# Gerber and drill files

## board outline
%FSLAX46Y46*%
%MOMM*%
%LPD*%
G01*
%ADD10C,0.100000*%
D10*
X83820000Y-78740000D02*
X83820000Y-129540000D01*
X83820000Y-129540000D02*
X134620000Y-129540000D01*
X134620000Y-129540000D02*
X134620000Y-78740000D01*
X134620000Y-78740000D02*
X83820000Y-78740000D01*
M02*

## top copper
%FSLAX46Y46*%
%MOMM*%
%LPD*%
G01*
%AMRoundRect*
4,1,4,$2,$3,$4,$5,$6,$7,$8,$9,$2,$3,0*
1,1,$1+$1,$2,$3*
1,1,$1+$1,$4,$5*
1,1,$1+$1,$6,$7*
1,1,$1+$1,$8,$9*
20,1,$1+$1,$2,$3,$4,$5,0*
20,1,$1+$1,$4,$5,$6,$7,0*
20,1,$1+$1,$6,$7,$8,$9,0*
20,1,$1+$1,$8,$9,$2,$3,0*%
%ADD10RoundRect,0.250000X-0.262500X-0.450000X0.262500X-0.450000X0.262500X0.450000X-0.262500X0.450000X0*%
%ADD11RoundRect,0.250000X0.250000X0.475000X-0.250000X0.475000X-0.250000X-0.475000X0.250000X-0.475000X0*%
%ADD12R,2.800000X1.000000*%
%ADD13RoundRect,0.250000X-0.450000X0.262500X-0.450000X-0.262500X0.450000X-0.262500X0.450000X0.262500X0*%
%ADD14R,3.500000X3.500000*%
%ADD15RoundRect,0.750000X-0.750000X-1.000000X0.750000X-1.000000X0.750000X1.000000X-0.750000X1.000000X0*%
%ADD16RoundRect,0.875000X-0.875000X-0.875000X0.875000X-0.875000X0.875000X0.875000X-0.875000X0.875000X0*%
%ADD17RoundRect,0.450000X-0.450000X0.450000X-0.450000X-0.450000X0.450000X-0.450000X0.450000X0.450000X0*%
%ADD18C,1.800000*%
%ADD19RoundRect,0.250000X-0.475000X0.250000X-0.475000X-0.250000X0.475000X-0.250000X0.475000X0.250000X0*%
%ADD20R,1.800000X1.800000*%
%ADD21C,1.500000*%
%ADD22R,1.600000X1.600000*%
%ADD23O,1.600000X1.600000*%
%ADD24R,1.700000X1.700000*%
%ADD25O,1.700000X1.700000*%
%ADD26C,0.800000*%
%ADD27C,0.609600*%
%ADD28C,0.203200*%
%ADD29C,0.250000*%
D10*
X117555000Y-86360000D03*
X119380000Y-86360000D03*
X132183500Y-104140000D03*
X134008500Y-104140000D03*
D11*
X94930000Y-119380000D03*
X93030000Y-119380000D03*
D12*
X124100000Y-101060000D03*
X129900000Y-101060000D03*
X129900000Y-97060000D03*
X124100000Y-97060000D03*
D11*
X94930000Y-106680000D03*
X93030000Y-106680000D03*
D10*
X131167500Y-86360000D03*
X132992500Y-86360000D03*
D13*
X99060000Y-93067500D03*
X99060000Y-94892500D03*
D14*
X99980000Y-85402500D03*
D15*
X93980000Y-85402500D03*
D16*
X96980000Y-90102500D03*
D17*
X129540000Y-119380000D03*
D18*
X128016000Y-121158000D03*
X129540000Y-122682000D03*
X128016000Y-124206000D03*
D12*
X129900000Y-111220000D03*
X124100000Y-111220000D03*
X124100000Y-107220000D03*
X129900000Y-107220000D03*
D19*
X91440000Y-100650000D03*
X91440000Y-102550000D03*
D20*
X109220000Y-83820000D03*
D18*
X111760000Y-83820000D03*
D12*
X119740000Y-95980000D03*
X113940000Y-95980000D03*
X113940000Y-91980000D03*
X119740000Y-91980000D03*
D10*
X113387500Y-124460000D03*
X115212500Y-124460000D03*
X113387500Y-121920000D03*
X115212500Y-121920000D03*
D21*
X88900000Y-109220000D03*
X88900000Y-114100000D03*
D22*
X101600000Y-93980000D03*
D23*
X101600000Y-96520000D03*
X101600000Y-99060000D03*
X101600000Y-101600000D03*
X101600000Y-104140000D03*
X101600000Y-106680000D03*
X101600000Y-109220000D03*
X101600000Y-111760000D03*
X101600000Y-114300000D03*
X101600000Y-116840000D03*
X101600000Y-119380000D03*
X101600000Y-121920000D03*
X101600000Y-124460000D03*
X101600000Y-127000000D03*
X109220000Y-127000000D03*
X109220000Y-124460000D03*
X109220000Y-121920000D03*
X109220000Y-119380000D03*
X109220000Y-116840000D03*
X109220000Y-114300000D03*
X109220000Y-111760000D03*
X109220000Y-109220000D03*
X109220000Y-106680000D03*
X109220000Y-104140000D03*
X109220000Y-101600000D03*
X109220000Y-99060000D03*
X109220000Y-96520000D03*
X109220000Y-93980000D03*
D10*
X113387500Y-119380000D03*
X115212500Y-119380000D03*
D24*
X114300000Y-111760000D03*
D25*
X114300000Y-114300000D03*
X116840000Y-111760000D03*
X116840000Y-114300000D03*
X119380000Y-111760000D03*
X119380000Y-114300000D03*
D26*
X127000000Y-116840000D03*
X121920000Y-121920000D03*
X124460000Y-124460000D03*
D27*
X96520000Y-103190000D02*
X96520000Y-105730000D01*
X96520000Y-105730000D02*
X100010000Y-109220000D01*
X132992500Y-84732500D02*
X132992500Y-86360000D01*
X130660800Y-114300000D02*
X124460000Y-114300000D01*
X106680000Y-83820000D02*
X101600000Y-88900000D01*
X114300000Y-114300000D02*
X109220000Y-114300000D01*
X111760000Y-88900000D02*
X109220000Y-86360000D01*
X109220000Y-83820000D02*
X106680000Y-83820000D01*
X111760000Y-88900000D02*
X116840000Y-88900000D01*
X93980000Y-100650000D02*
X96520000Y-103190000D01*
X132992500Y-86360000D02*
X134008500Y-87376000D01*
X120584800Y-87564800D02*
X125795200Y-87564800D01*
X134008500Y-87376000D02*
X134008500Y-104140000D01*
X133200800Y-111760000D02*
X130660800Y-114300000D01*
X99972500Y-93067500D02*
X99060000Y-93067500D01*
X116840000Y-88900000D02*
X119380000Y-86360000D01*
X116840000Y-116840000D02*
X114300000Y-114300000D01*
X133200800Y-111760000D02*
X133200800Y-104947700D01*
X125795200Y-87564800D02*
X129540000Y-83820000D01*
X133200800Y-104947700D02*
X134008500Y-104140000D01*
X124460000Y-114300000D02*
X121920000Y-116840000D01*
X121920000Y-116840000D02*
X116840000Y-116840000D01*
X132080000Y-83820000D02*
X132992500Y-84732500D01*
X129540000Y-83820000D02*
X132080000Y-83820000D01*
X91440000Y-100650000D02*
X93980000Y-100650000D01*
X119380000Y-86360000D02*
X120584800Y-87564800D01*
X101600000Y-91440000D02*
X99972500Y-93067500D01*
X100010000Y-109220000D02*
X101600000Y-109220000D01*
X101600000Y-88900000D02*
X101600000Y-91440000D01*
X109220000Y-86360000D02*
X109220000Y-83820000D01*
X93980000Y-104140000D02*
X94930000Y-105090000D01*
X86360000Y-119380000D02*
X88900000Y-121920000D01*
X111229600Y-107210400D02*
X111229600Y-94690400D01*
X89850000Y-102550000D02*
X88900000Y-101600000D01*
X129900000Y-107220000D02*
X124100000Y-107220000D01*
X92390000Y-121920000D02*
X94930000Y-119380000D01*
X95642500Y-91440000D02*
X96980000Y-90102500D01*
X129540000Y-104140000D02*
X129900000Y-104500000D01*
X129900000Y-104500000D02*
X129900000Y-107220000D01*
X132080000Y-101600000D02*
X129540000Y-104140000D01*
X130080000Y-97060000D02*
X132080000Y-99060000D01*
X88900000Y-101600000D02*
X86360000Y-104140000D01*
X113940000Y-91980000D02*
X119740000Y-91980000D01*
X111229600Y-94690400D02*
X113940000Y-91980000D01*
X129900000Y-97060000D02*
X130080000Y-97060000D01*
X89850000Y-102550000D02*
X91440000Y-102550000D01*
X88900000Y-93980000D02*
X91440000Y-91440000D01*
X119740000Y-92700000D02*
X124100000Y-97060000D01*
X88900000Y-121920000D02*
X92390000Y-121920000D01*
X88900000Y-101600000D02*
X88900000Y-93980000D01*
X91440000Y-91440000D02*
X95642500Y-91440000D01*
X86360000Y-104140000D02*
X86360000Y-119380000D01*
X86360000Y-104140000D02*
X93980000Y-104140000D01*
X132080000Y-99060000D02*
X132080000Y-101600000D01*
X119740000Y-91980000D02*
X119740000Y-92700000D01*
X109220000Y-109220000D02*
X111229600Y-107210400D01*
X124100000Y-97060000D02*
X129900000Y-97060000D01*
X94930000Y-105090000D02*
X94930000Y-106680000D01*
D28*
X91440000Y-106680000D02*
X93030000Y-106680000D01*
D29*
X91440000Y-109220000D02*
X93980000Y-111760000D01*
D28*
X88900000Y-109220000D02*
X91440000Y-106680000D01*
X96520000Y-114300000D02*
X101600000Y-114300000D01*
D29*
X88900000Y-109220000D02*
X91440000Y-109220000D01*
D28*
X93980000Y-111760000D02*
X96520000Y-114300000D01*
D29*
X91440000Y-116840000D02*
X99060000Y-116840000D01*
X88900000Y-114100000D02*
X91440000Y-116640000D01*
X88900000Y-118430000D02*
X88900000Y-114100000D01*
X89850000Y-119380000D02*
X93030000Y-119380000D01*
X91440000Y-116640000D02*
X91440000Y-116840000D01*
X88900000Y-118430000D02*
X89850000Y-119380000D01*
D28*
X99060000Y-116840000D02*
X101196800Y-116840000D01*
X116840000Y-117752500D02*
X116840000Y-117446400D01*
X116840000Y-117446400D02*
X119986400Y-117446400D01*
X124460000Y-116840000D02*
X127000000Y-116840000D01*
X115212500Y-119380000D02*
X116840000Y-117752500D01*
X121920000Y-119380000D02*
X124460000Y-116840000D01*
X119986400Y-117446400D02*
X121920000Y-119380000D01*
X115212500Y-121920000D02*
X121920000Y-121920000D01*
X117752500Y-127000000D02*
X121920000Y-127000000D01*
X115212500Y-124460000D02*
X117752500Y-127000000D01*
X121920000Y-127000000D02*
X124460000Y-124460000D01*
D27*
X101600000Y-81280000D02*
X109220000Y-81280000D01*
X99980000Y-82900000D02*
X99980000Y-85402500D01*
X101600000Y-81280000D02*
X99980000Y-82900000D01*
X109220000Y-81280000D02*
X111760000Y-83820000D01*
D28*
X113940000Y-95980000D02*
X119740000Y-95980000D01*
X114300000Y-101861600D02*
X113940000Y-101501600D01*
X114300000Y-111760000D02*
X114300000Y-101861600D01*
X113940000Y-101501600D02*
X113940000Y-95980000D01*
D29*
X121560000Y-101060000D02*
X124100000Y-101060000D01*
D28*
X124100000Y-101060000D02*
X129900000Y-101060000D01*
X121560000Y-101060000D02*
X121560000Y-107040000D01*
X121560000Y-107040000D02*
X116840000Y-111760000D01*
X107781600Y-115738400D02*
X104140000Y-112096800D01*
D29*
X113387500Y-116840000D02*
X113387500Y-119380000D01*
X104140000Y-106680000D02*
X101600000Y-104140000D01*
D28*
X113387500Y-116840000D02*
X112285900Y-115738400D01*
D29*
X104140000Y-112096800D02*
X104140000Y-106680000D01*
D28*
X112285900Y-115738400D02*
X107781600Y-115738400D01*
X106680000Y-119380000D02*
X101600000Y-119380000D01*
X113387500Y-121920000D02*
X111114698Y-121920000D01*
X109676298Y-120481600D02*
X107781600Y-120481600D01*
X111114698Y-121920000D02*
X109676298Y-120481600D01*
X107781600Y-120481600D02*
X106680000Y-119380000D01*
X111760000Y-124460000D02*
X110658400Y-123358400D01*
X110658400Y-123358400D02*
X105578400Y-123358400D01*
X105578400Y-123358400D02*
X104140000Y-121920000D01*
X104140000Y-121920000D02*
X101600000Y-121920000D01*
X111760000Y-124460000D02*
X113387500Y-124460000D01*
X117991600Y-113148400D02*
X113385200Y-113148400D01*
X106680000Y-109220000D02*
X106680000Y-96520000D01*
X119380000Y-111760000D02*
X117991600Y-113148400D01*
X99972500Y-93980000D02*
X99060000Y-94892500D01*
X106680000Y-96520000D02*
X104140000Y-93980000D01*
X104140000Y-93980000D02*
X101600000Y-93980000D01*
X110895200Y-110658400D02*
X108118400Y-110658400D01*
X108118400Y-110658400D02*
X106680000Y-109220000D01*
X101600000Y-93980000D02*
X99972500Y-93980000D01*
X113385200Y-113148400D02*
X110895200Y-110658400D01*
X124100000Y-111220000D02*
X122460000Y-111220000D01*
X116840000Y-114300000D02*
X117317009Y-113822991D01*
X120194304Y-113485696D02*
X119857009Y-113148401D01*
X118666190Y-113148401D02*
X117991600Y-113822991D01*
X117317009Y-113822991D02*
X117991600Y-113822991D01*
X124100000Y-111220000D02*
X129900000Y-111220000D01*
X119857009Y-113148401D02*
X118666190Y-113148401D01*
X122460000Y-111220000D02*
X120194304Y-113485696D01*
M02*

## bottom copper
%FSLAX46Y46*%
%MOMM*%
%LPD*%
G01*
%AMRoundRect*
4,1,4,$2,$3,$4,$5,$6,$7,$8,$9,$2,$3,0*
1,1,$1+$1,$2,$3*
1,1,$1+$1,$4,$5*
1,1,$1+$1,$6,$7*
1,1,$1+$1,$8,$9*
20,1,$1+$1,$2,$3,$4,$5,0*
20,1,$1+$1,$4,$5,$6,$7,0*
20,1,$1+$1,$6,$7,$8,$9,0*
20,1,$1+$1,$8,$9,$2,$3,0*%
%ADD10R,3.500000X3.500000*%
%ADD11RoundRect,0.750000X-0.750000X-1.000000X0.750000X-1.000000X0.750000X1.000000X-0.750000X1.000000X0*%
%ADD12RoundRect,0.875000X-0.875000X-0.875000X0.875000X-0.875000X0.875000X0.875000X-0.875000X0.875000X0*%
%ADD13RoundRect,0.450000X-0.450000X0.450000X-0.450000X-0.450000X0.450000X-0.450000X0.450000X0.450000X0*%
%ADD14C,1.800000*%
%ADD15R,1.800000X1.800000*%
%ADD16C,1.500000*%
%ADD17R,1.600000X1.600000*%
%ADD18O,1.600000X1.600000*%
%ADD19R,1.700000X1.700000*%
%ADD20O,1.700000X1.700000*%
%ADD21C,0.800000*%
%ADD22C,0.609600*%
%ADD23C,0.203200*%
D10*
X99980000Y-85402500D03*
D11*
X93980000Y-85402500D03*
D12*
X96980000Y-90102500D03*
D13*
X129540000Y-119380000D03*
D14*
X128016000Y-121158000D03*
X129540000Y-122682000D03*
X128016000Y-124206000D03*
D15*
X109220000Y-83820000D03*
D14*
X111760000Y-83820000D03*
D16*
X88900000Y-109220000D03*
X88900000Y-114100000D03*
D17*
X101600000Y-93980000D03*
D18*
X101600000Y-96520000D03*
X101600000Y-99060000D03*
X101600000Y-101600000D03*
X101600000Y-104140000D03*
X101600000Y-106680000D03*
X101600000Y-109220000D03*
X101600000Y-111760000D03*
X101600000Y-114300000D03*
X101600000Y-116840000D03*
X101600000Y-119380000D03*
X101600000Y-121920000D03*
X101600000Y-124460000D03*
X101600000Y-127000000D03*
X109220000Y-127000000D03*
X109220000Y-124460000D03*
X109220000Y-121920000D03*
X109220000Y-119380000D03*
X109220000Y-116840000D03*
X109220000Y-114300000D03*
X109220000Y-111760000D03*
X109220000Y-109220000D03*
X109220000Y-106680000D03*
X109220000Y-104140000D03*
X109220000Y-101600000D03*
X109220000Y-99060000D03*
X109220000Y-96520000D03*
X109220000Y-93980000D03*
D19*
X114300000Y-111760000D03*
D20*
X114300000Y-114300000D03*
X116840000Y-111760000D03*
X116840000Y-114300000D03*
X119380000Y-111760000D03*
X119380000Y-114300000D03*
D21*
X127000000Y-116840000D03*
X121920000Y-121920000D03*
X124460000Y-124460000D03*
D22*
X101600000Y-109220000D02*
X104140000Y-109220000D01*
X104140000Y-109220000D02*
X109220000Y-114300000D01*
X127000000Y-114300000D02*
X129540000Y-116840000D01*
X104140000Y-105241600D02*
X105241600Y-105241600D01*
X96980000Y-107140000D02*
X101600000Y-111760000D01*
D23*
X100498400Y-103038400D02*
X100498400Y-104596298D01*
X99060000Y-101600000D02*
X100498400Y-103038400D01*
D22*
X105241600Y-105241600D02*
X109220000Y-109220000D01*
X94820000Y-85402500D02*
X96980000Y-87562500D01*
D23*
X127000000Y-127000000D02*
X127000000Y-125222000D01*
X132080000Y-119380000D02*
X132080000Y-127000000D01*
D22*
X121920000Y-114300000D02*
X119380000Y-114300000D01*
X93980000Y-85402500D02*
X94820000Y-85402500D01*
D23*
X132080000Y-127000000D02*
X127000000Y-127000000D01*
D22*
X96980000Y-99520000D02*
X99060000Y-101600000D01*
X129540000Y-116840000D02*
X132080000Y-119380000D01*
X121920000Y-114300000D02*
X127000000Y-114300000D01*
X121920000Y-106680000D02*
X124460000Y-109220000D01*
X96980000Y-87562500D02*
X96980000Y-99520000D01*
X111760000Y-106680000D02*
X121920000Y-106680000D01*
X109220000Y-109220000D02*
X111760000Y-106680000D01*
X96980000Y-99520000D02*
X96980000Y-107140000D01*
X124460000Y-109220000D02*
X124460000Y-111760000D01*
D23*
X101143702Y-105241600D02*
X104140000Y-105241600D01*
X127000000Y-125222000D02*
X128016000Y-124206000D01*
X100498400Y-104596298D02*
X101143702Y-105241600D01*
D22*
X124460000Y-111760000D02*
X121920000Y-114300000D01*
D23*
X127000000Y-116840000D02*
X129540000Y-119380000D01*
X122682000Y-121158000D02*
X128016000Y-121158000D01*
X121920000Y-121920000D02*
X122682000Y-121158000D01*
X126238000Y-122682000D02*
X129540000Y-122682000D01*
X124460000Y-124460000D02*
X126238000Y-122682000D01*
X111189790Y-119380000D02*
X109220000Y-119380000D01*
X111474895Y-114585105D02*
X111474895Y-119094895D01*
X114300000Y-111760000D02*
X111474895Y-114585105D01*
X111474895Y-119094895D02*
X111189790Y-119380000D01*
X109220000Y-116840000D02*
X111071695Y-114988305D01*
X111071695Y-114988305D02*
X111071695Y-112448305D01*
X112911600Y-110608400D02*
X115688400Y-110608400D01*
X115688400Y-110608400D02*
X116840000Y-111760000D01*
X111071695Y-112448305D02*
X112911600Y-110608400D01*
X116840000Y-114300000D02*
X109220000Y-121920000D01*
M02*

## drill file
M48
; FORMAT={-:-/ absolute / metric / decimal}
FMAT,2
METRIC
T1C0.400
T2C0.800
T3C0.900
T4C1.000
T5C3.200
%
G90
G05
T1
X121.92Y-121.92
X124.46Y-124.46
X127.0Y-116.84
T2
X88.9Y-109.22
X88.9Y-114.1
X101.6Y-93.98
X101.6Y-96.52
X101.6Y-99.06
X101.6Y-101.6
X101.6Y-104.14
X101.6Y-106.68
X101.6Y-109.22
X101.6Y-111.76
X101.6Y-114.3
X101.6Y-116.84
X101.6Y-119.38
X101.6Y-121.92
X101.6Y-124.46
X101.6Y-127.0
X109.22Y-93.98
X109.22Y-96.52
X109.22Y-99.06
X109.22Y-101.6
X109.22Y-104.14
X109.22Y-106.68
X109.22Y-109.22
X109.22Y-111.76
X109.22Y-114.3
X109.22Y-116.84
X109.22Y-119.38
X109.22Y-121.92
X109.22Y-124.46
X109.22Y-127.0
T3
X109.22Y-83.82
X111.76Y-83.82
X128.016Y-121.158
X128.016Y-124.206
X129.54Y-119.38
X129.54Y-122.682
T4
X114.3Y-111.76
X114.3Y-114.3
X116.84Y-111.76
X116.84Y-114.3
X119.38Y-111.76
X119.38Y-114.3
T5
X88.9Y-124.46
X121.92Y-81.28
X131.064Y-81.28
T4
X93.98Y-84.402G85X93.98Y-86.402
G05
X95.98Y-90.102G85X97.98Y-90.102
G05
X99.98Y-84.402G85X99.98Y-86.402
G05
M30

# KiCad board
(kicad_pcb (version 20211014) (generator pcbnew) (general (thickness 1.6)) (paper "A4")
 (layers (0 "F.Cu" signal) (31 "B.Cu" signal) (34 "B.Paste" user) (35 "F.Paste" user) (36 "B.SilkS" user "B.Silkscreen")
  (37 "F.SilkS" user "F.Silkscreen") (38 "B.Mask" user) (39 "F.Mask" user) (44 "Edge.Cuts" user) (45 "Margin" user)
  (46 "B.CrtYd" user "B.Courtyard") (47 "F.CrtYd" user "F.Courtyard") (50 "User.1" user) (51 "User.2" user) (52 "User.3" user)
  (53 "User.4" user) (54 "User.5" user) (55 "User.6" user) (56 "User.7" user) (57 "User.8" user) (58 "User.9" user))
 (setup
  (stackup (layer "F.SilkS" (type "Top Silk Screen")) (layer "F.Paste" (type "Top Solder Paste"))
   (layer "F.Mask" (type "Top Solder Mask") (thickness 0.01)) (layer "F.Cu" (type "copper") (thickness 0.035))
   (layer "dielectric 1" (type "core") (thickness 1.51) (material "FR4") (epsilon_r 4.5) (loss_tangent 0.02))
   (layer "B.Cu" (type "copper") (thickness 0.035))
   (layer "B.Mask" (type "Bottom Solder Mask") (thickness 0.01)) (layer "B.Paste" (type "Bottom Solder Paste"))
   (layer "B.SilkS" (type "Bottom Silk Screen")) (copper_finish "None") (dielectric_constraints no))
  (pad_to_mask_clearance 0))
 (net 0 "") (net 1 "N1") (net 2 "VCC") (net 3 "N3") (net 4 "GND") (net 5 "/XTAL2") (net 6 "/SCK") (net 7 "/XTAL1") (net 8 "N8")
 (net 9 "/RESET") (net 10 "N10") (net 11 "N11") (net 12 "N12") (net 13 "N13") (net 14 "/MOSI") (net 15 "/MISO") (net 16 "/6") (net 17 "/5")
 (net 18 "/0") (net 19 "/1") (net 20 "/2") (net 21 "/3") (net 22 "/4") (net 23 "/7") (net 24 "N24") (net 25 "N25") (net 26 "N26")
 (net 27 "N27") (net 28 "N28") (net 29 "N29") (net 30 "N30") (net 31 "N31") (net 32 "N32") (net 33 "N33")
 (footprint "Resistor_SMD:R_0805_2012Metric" (layer "F.Cu") (at 118.4675 86.36)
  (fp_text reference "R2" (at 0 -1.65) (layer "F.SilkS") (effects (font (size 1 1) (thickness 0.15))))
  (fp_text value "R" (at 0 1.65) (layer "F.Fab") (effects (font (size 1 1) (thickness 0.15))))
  (pad "1" smd roundrect (at -0.9125 0) (size 1.025 1.4) (layers "F.Cu" "F.Paste" "F.Mask") (roundrect_rratio 0.243902) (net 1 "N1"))
  (pad "2" smd roundrect (at 0.9125 0) (size 1.025 1.4) (layers "F.Cu" "F.Paste" "F.Mask") (roundrect_rratio 0.243902) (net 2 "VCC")))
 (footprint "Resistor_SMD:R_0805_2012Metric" (layer "F.Cu") (at 133.096 104.14)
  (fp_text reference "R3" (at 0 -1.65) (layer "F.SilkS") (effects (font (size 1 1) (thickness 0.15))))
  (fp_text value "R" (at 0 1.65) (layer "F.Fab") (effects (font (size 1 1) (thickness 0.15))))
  (pad "1" smd roundrect (at -0.9125 0) (size 1.025 1.4) (layers "F.Cu" "F.Paste" "F.Mask") (roundrect_rratio 0.243902) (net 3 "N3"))
  (pad "2" smd roundrect (at 0.9125 0) (size 1.025 1.4) (layers "F.Cu" "F.Paste" "F.Mask") (roundrect_rratio 0.243902) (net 2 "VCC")))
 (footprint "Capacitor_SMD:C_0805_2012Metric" (layer "F.Cu") (at 93.98 119.38 180)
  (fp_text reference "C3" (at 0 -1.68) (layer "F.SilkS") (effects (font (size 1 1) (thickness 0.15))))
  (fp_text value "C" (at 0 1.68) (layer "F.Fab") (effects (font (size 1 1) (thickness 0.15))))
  (pad "1" smd roundrect (at -0.95 0 180) (size 1 1.45) (layers "F.Cu" "F.Paste" "F.Mask") (roundrect_rratio 0.25) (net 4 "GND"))
  (pad "2" smd roundrect (at 0.95 0 180) (size 1 1.45) (layers "F.Cu" "F.Paste" "F.Mask") (roundrect_rratio 0.25) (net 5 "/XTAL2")))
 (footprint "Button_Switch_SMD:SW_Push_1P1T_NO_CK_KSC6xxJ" (layer "F.Cu") (at 127 99.06 180)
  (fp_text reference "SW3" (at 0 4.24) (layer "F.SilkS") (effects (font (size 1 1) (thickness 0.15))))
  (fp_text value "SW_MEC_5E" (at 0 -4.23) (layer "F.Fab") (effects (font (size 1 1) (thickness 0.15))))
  (pad "1" smd rect (at 2.9 -2 180) (size 2.8 1) (layers "F.Cu" "F.Paste" "F.Mask") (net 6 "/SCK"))
  (pad "1" smd rect (at -2.9 -2 180) (size 2.8 1) (layers "F.Cu" "F.Paste" "F.Mask") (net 6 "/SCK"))
  (pad "2" smd rect (at -2.9 2 180) (size 2.8 1) (layers "F.Cu" "F.Paste" "F.Mask") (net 4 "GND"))
  (pad "2" smd rect (at 2.9 2 180) (size 2.8 1) (layers "F.Cu" "F.Paste" "F.Mask") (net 4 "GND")))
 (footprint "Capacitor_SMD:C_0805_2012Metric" (layer "F.Cu") (at 93.98 106.68 180)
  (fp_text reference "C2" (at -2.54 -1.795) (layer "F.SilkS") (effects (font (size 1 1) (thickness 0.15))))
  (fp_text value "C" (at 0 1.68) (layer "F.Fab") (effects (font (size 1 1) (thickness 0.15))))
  (pad "1" smd roundrect (at -0.95 0 180) (size 1 1.45) (layers "F.Cu" "F.Paste" "F.Mask") (roundrect_rratio 0.25) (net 4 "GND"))
  (pad "2" smd roundrect (at 0.95 0 180) (size 1 1.45) (layers "F.Cu" "F.Paste" "F.Mask") (roundrect_rratio 0.25) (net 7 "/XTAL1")))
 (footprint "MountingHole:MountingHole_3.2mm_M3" (layer "F.Cu") (at 121.92 81.28)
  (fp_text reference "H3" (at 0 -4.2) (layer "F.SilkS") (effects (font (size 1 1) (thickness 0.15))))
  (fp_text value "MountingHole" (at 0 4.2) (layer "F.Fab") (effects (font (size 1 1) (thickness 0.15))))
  (pad "" np_thru_hole circle (at 0 0) (size 3.2 3.2) (drill 3.2) (layers *.Cu *.Mask)))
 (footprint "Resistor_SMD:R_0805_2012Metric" (layer "F.Cu") (at 132.08 86.36)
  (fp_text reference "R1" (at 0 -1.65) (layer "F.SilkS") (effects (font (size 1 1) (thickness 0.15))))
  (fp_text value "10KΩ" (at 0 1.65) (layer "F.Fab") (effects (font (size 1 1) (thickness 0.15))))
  (pad "1" smd roundrect (at -0.9125 0) (size 1.025 1.4) (layers "F.Cu" "F.Paste" "F.Mask") (roundrect_rratio 0.243902) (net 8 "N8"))
  (pad "2" smd roundrect (at 0.9125 0) (size 1.025 1.4) (layers "F.Cu" "F.Paste" "F.Mask") (roundrect_rratio 0.243902) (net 2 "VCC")))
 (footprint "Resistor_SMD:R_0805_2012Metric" (layer "F.Cu") (at 99.06 93.98 -90)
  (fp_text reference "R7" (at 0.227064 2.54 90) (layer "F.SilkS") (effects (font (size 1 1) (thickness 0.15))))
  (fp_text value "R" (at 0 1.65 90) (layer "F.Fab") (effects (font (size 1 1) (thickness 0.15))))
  (pad "1" smd roundrect (at -0.9125 0 270) (size 1.025 1.4) (layers "F.Cu" "F.Paste" "F.Mask") (roundrect_rratio 0.243902) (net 2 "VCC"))
  (pad "2" smd roundrect (at 0.9125 0 270) (size 1.025 1.4) (layers "F.Cu" "F.Paste" "F.Mask") (roundrect_rratio 0.243902) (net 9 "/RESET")))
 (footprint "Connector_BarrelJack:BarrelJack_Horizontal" (layer "F.Cu") (at 99.98 85.4025)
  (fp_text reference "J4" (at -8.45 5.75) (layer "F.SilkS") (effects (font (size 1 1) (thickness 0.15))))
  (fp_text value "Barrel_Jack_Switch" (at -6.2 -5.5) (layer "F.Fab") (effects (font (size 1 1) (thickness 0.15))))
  (pad "1" thru_hole rect (at 0 0) (size 3.5 3.5) (drill oval 1 3) (layers *.Cu *.Mask) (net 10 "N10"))
  (pad "2" thru_hole roundrect (at -6 0) (size 3 3.5) (drill oval 1 3) (layers *.Cu *.Mask) (roundrect_rratio 0.25) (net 4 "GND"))
  (pad "3" thru_hole roundrect (at -3 4.7) (size 3.5 3.5) (drill oval 3 1) (layers *.Cu *.Mask) (roundrect_rratio 0.25) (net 4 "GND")))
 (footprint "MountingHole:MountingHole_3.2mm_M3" (layer "F.Cu") (at 88.9 124.46)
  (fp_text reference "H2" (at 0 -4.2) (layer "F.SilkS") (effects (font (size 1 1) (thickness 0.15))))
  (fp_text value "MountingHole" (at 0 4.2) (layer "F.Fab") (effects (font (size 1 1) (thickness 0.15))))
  (pad "" np_thru_hole circle (at 0 0) (size 3.2 3.2) (drill 3.2) (layers *.Cu *.Mask)))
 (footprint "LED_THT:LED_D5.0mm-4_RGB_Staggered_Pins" (layer "F.Cu") (at 129.54 119.38 -90)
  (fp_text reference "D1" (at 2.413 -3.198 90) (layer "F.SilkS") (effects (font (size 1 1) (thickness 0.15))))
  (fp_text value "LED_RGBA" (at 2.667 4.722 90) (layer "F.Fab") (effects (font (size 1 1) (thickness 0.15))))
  (pad "1" thru_hole roundrect (at 0 0 270) (size 1.8 1.8) (drill 0.9) (layers *.Cu *.Mask) (roundrect_rratio 0.25) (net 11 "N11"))
  (pad "2" thru_hole circle (at 1.778 1.524 270) (size 1.8 1.8) (drill 0.9) (layers *.Cu *.Mask) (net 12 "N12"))
  (pad "3" thru_hole circle (at 3.302 0 270) (size 1.8 1.8) (drill 0.9) (layers *.Cu *.Mask) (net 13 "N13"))
  (pad "4" thru_hole circle (at 4.826 1.524 270) (size 1.8 1.8) (drill 0.9) (layers *.Cu *.Mask) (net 4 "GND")))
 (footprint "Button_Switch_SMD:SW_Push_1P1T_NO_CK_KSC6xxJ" (layer "F.Cu") (at 127 109.22 180)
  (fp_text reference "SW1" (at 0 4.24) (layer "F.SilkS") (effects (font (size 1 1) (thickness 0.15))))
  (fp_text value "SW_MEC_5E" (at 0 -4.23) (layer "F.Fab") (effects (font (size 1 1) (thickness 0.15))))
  (pad "1" smd rect (at -2.9 -2 180) (size 2.8 1) (layers "F.Cu" "F.Paste" "F.Mask") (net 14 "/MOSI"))
  (pad "1" smd rect (at 2.9 -2 180) (size 2.8 1) (layers "F.Cu" "F.Paste" "F.Mask") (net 14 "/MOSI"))
  (pad "2" smd rect (at 2.9 2 180) (size 2.8 1) (layers "F.Cu" "F.Paste" "F.Mask") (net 4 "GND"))
  (pad "2" smd rect (at -2.9 2 180) (size 2.8 1) (layers "F.Cu" "F.Paste" "F.Mask") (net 4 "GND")))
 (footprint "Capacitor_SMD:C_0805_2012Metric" (layer "F.Cu") (at 91.44 101.6 -90)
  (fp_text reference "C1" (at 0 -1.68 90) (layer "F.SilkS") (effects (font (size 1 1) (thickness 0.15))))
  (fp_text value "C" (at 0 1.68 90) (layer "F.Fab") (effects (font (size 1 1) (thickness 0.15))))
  (pad "1" smd roundrect (at -0.95 0 270) (size 1 1.45) (layers "F.Cu" "F.Paste" "F.Mask") (roundrect_rratio 0.25) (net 2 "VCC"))
  (pad "2" smd roundrect (at 0.95 0 270) (size 1 1.45) (layers "F.Cu" "F.Paste" "F.Mask") (roundrect_rratio 0.25) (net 4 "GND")))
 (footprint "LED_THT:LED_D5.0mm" (layer "F.Cu") (at 109.22 83.82)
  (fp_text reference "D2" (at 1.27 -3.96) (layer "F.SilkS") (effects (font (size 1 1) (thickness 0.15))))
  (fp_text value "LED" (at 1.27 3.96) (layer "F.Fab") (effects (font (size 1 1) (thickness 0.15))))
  (pad "1" thru_hole rect (at 0 0) (size 1.8 1.8) (drill 0.9) (layers *.Cu *.Mask) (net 2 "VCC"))
  (pad "2" thru_hole circle (at 2.54 0) (size 1.8 1.8) (drill 0.9) (layers *.Cu *.Mask) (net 10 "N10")))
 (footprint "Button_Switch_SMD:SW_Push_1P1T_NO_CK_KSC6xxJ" (layer "F.Cu") (at 116.84 93.98 180)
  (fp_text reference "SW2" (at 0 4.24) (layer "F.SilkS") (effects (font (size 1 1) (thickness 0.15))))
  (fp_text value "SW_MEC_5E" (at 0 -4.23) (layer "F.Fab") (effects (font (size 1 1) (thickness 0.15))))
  (pad "1" smd rect (at -2.9 -2 180) (size 2.8 1) (layers "F.Cu" "F.Paste" "F.Mask") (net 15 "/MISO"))
  (pad "1" smd rect (at 2.9 -2 180) (size 2.8 1) (layers "F.Cu" "F.Paste" "F.Mask") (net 15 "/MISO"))
  (pad "2" smd rect (at 2.9 2 180) (size 2.8 1) (layers "F.Cu" "F.Paste" "F.Mask") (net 4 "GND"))
  (pad "2" smd rect (at -2.9 2 180) (size 2.8 1) (layers "F.Cu" "F.Paste" "F.Mask") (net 4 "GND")))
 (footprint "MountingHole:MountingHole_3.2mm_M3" (layer "F.Cu") (at 131.064 81.28)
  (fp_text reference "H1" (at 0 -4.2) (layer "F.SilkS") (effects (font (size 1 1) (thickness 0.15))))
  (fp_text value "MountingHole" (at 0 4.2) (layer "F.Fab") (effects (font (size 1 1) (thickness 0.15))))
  (pad "" np_thru_hole circle (at 0 0) (size 3.2 3.2) (drill 3.2) (layers *.Cu *.Mask)))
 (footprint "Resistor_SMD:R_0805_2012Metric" (layer "F.Cu") (at 114.3 124.46)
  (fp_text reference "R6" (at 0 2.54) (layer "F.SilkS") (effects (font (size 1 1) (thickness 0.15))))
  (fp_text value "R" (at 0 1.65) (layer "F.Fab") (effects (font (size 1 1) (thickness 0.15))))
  (pad "1" smd roundrect (at -0.9125 0) (size 1.025 1.4) (layers "F.Cu" "F.Paste" "F.Mask") (roundrect_rratio 0.243902) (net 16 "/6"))
  (pad "2" smd roundrect (at 0.9125 0) (size 1.025 1.4) (layers "F.Cu" "F.Paste" "F.Mask") (roundrect_rratio 0.243902) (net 13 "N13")))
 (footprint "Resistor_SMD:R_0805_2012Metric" (layer "F.Cu") (at 114.3 121.92)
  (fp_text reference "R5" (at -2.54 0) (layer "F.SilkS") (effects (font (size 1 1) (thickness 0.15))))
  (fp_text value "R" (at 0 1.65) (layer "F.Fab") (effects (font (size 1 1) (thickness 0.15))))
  (pad "1" smd roundrect (at -0.9125 0) (size 1.025 1.4) (layers "F.Cu" "F.Paste" "F.Mask") (roundrect_rratio 0.243902) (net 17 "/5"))
  (pad "2" smd roundrect (at 0.9125 0) (size 1.025 1.4) (layers "F.Cu" "F.Paste" "F.Mask") (roundrect_rratio 0.243902) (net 12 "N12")))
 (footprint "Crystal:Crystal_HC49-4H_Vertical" (layer "F.Cu") (at 88.9 109.22 -90)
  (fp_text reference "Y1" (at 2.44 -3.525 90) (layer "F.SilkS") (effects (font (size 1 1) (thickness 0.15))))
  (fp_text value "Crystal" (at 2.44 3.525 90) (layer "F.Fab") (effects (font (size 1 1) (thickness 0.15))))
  (pad "1" thru_hole circle (at 0 0 270) (size 1.5 1.5) (drill 0.8) (layers *.Cu *.Mask) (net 7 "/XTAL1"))
  (pad "2" thru_hole circle (at 4.88 0 270) (size 1.5 1.5) (drill 0.8) (layers *.Cu *.Mask) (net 5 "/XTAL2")))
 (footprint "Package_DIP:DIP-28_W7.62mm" (layer "F.Cu") (at 101.6 93.98)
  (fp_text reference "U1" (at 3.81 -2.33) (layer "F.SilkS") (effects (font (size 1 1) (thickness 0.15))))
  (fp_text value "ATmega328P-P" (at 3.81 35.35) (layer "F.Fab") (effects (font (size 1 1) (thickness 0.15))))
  (pad "1" thru_hole rect (at 0 0) (size 1.6 1.6) (drill 0.8) (layers *.Cu *.Mask) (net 9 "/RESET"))
  (pad "2" thru_hole oval (at 0 2.54) (size 1.6 1.6) (drill 0.8) (layers *.Cu *.Mask) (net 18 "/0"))
  (pad "3" thru_hole oval (at 0 5.08) (size 1.6 1.6) (drill 0.8) (layers *.Cu *.Mask) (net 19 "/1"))
  (pad "4" thru_hole oval (at 0 7.62) (size 1.6 1.6) (drill 0.8) (layers *.Cu *.Mask) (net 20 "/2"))
  (pad "5" thru_hole oval (at 0 10.16) (size 1.6 1.6) (drill 0.8) (layers *.Cu *.Mask) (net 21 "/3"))
  (pad "6" thru_hole oval (at 0 12.7) (size 1.6 1.6) (drill 0.8) (layers *.Cu *.Mask) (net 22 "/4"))
  (pad "7" thru_hole oval (at 0 15.24) (size 1.6 1.6) (drill 0.8) (layers *.Cu *.Mask) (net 2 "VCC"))
  (pad "8" thru_hole oval (at 0 17.78) (size 1.6 1.6) (drill 0.8) (layers *.Cu *.Mask) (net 4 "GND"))
  (pad "9" thru_hole oval (at 0 20.32) (size 1.6 1.6) (drill 0.8) (layers *.Cu *.Mask) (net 7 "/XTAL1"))
  (pad "10" thru_hole oval (at 0 22.86) (size 1.6 1.6) (drill 0.8) (layers *.Cu *.Mask) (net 5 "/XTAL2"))
  (pad "11" thru_hole oval (at 0 25.4) (size 1.6 1.6) (drill 0.8) (layers *.Cu *.Mask) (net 17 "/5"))
  (pad "12" thru_hole oval (at 0 27.94) (size 1.6 1.6) (drill 0.8) (layers *.Cu *.Mask) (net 16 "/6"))
  (pad "13" thru_hole oval (at 0 30.48) (size 1.6 1.6) (drill 0.8) (layers *.Cu *.Mask) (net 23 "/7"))
  (pad "14" thru_hole oval (at 0 33.02) (size 1.6 1.6) (drill 0.8) (layers *.Cu *.Mask) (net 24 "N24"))
  (pad "15" thru_hole oval (at 7.62 33.02) (size 1.6 1.6) (drill 0.8) (layers *.Cu *.Mask) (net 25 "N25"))
  (pad "16" thru_hole oval (at 7.62 30.48) (size 1.6 1.6) (drill 0.8) (layers *.Cu *.Mask) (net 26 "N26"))
  (pad "17" thru_hole oval (at 7.62 27.94) (size 1.6 1.6) (drill 0.8) (layers *.Cu *.Mask) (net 14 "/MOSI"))
  (pad "18" thru_hole oval (at 7.62 25.4) (size 1.6 1.6) (drill 0.8) (layers *.Cu *.Mask) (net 15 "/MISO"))
  (pad "19" thru_hole oval (at 7.62 22.86) (size 1.6 1.6) (drill 0.8) (layers *.Cu *.Mask) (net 6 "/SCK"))
  (pad "20" thru_hole oval (at 7.62 20.32) (size 1.6 1.6) (drill 0.8) (layers *.Cu *.Mask) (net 2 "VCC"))
  (pad "21" thru_hole oval (at 7.62 17.78) (size 1.6 1.6) (drill 0.8) (layers *.Cu *.Mask) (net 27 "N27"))
  (pad "22" thru_hole oval (at 7.62 15.24) (size 1.6 1.6) (drill 0.8) (layers *.Cu *.Mask) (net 4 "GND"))
  (pad "23" thru_hole oval (at 7.62 12.7) (size 1.6 1.6) (drill 0.8) (layers *.Cu *.Mask) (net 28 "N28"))
  (pad "24" thru_hole oval (at 7.62 10.16) (size 1.6 1.6) (drill 0.8) (layers *.Cu *.Mask) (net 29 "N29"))
  (pad "25" thru_hole oval (at 7.62 7.62) (size 1.6 1.6) (drill 0.8) (layers *.Cu *.Mask) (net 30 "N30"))
  (pad "26" thru_hole oval (at 7.62 5.08) (size 1.6 1.6) (drill 0.8) (layers *.Cu *.Mask) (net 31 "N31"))
  (pad "27" thru_hole oval (at 7.62 2.54) (size 1.6 1.6) (drill 0.8) (layers *.Cu *.Mask) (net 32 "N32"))
  (pad "28" thru_hole oval (at 7.62 0) (size 1.6 1.6) (drill 0.8) (layers *.Cu *.Mask) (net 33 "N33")))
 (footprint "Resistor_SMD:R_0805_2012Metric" (layer "F.Cu") (at 114.3 119.38)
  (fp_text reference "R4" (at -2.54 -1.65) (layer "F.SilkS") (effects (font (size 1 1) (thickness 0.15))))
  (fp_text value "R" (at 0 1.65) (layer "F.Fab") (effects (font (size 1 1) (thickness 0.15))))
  (pad "1" smd roundrect (at -0.9125 0) (size 1.025 1.4) (layers "F.Cu" "F.Paste" "F.Mask") (roundrect_rratio 0.243902) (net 21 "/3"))
  (pad "2" smd roundrect (at 0.9125 0) (size 1.025 1.4) (layers "F.Cu" "F.Paste" "F.Mask") (roundrect_rratio 0.243902) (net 11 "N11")))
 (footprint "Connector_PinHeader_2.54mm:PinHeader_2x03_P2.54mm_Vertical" (layer "B.Cu") (at 114.3 111.76 -90)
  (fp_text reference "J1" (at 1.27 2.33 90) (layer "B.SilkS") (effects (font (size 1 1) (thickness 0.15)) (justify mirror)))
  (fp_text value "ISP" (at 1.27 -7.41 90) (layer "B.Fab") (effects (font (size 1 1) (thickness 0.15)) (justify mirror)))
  (pad "1" thru_hole rect (at 0 0 270) (size 1.7 1.7) (drill 1) (layers *.Cu *.Mask) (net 15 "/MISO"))
  (pad "2" thru_hole oval (at 2.54 0 270) (size 1.7 1.7) (drill 1) (layers *.Cu *.Mask) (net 2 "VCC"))
  (pad "3" thru_hole oval (at 0 -2.54 270) (size 1.7 1.7) (drill 1) (layers *.Cu *.Mask) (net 6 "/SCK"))
  (pad "4" thru_hole oval (at 2.54 -2.54 270) (size 1.7 1.7) (drill 1) (layers *.Cu *.Mask) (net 14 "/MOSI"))
  (pad "5" thru_hole oval (at 0 -5.08 270) (size 1.7 1.7) (drill 1) (layers *.Cu *.Mask) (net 9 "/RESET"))
  (pad "6" thru_hole oval (at 2.54 -5.08 270) (size 1.7 1.7) (drill 1) (layers *.Cu *.Mask) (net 4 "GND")))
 (gr_line (start 83.82 78.74) (end 83.82 129.54) (layer "Edge.Cuts") (width 0.1))
 (gr_line (start 83.82 129.54) (end 134.62 129.54) (layer "Edge.Cuts") (width 0.1))
 (gr_line (start 134.62 129.54) (end 134.62 78.74) (layer "Edge.Cuts") (width 0.1))
 (gr_line (start 134.62 78.74) (end 83.82 78.74) (layer "Edge.Cuts") (width 0.1))
 (segment (start 96.52 103.19) (end 96.52 105.73) (width 0.6096) (layer "F.Cu") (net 2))
 (segment (start 96.52 105.73) (end 100.01 109.22) (width 0.6096) (layer "F.Cu") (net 2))
 (segment (start 132.9925 84.7325) (end 132.9925 86.36) (width 0.6096) (layer "F.Cu") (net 2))
 (segment (start 130.6608 114.3) (end 124.46 114.3) (width 0.6096) (layer "F.Cu") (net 2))
 (segment (start 106.68 83.82) (end 101.6 88.9) (width 0.6096) (layer "F.Cu") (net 2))
 (segment (start 114.3 114.3) (end 109.22 114.3) (width 0.6096) (layer "F.Cu") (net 2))
 (segment (start 111.76 88.9) (end 109.22 86.36) (width 0.6096) (layer "F.Cu") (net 2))
 (segment (start 109.22 83.82) (end 106.68 83.82) (width 0.6096) (layer "F.Cu") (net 2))
 (segment (start 111.76 88.9) (end 116.84 88.9) (width 0.6096) (layer "F.Cu") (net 2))
 (segment (start 93.98 100.65) (end 96.52 103.19) (width 0.6096) (layer "F.Cu") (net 2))
 (segment (start 132.9925 86.36) (end 134.0085 87.376) (width 0.6096) (layer "F.Cu") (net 2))
 (segment (start 120.5848 87.5648) (end 125.7952 87.5648) (width 0.6096) (layer "F.Cu") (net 2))
 (segment (start 134.0085 87.376) (end 134.0085 104.14) (width 0.6096) (layer "F.Cu") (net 2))
 (segment (start 133.2008 111.76) (end 130.6608 114.3) (width 0.6096) (layer "F.Cu") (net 2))
 (segment (start 99.9725 93.0675) (end 99.06 93.0675) (width 0.6096) (layer "F.Cu") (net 2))
 (segment (start 116.84 88.9) (end 119.38 86.36) (width 0.6096) (layer "F.Cu") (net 2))
 (segment (start 116.84 116.84) (end 114.3 114.3) (width 0.6096) (layer "F.Cu") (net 2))
 (segment (start 133.2008 111.76) (end 133.2008 104.9477) (width 0.6096) (layer "F.Cu") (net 2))
 (segment (start 125.7952 87.5648) (end 129.54 83.82) (width 0.6096) (layer "F.Cu") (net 2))
 (segment (start 133.2008 104.9477) (end 134.0085 104.14) (width 0.6096) (layer "F.Cu") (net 2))
 (segment (start 124.46 114.3) (end 121.92 116.84) (width 0.6096) (layer "F.Cu") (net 2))
 (segment (start 121.92 116.84) (end 116.84 116.84) (width 0.6096) (layer "F.Cu") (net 2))
 (segment (start 132.08 83.82) (end 132.9925 84.7325) (width 0.6096) (layer "F.Cu") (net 2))
 (segment (start 129.54 83.82) (end 132.08 83.82) (width 0.6096) (layer "F.Cu") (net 2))
 (segment (start 91.44 100.65) (end 93.98 100.65) (width 0.6096) (layer "F.Cu") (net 2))
 (segment (start 119.38 86.36) (end 120.5848 87.5648) (width 0.6096) (layer "F.Cu") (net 2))
 (segment (start 101.6 91.44) (end 99.9725 93.0675) (width 0.6096) (layer "F.Cu") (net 2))
 (segment (start 100.01 109.22) (end 101.6 109.22) (width 0.6096) (layer "F.Cu") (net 2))
 (segment (start 101.6 88.9) (end 101.6 91.44) (width 0.6096) (layer "F.Cu") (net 2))
 (segment (start 109.22 86.36) (end 109.22 83.82) (width 0.6096) (layer "F.Cu") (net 2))
 (segment (start 101.6 109.22) (end 104.14 109.22) (width 0.6096) (layer "B.Cu") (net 2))
 (segment (start 104.14 109.22) (end 109.22 114.3) (width 0.6096) (layer "B.Cu") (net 2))
 (segment (start 93.98 104.14) (end 94.93 105.09) (width 0.6096) (layer "F.Cu") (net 4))
 (segment (start 86.36 119.38) (end 88.9 121.92) (width 0.6096) (layer "F.Cu") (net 4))
 (segment (start 111.2296 107.2104) (end 111.2296 94.6904) (width 0.6096) (layer "F.Cu") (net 4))
 (segment (start 89.85 102.55) (end 88.9 101.6) (width 0.6096) (layer "F.Cu") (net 4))
 (segment (start 129.9 107.22) (end 124.1 107.22) (width 0.6096) (layer "F.Cu") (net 4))
 (segment (start 92.39 121.92) (end 94.93 119.38) (width 0.6096) (layer "F.Cu") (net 4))
 (segment (start 95.6425 91.44) (end 96.98 90.1025) (width 0.6096) (layer "F.Cu") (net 4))
 (segment (start 129.54 104.14) (end 129.9 104.5) (width 0.6096) (layer "F.Cu") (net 4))
 (segment (start 129.9 104.5) (end 129.9 107.22) (width 0.6096) (layer "F.Cu") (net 4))
 (segment (start 132.08 101.6) (end 129.54 104.14) (width 0.6096) (layer "F.Cu") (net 4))
 (segment (start 130.08 97.06) (end 132.08 99.06) (width 0.6096) (layer "F.Cu") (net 4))
 (segment (start 88.9 101.6) (end 86.36 104.14) (width 0.6096) (layer "F.Cu") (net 4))
 (segment (start 113.94 91.98) (end 119.74 91.98) (width 0.6096) (layer "F.Cu") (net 4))
 (segment (start 111.2296 94.6904) (end 113.94 91.98) (width 0.6096) (layer "F.Cu") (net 4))
 (segment (start 129.9 97.06) (end 130.08 97.06) (width 0.6096) (layer "F.Cu") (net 4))
 (segment (start 89.85 102.55) (end 91.44 102.55) (width 0.6096) (layer "F.Cu") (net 4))
 (segment (start 88.9 93.98) (end 91.44 91.44) (width 0.6096) (layer "F.Cu") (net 4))
 (segment (start 119.74 92.7) (end 124.1 97.06) (width 0.6096) (layer "F.Cu") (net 4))
 (segment (start 88.9 121.92) (end 92.39 121.92) (width 0.6096) (layer "F.Cu") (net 4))
 (segment (start 88.9 101.6) (end 88.9 93.98) (width 0.6096) (layer "F.Cu") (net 4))
 (segment (start 91.44 91.44) (end 95.6425 91.44) (width 0.6096) (layer "F.Cu") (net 4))
 (segment (start 86.36 104.14) (end 86.36 119.38) (width 0.6096) (layer "F.Cu") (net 4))
 (segment (start 86.36 104.14) (end 93.98 104.14) (width 0.6096) (layer "F.Cu") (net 4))
 (segment (start 132.08 99.06) (end 132.08 101.6) (width 0.6096) (layer "F.Cu") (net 4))
 (segment (start 119.74 91.98) (end 119.74 92.7) (width 0.6096) (layer "F.Cu") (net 4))
 (segment (start 109.22 109.22) (end 111.2296 107.2104) (width 0.6096) (layer "F.Cu") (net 4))
 (segment (start 124.1 97.06) (end 129.9 97.06) (width 0.6096) (layer "F.Cu") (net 4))
 (segment (start 94.93 105.09) (end 94.93 106.68) (width 0.6096) (layer "F.Cu") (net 4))
 (segment (start 127 114.3) (end 129.54 116.84) (width 0.6096) (layer "B.Cu") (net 4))
 (segment (start 104.14 105.2416) (end 105.2416 105.2416) (width 0.6096) (layer "B.Cu") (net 4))
 (segment (start 96.98 107.14) (end 101.6 111.76) (width 0.6096) (layer "B.Cu") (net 4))
 (segment (start 100.4984 103.0384) (end 100.4984 104.596298) (width 0.2032) (layer "B.Cu") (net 4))
 (segment (start 99.06 101.6) (end 100.4984 103.0384) (width 0.2032) (layer "B.Cu") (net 4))
 (segment (start 105.2416 105.2416) (end 109.22 109.22) (width 0.6096) (layer "B.Cu") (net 4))
 (segment (start 94.82 85.4025) (end 96.98 87.5625) (width 0.6096) (layer "B.Cu") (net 4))
 (segment (start 127 127) (end 127 125.222) (width 0.2032) (layer "B.Cu") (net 4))
 (segment (start 132.08 119.38) (end 132.08 127) (width 0.2032) (layer "B.Cu") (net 4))
 (segment (start 121.92 114.3) (end 119.38 114.3) (width 0.6096) (layer "B.Cu") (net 4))
 (segment (start 93.98 85.4025) (end 94.82 85.4025) (width 0.6096) (layer "B.Cu") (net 4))
 (segment (start 132.08 127) (end 127 127) (width 0.2032) (layer "B.Cu") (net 4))
 (segment (start 96.98 99.52) (end 99.06 101.6) (width 0.6096) (layer "B.Cu") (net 4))
 (segment (start 129.54 116.84) (end 132.08 119.38) (width 0.6096) (layer "B.Cu") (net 4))
 (segment (start 121.92 114.3) (end 127 114.3) (width 0.6096) (layer "B.Cu") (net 4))
 (segment (start 121.92 106.68) (end 124.46 109.22) (width 0.6096) (layer "B.Cu") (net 4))
 (segment (start 96.98 87.5625) (end 96.98 99.52) (width 0.6096) (layer "B.Cu") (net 4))
 (segment (start 111.76 106.68) (end 121.92 106.68) (width 0.6096) (layer "B.Cu") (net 4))
 (segment (start 109.22 109.22) (end 111.76 106.68) (width 0.6096) (layer "B.Cu") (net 4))
 (segment (start 96.98 99.52) (end 96.98 107.14) (width 0.6096) (layer "B.Cu") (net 4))
 (segment (start 124.46 109.22) (end 124.46 111.76) (width 0.6096) (layer "B.Cu") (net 4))
 (segment (start 101.143702 105.2416) (end 104.14 105.2416) (width 0.2032) (layer "B.Cu") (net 4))
 (segment (start 127 125.222) (end 128.016 124.206) (width 0.2032) (layer "B.Cu") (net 4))
 (segment (start 100.4984 104.596298) (end 101.143702 105.2416) (width 0.2032) (layer "B.Cu") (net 4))
 (segment (start 124.46 111.76) (end 121.92 114.3) (width 0.6096) (layer "B.Cu") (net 4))
 (segment (start 91.44 106.68) (end 93.03 106.68) (width 0.2032) (layer "F.Cu") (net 7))
 (segment (start 91.44 109.22) (end 93.98 111.76) (width 0.25) (layer "F.Cu") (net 7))
 (segment (start 88.9 109.22) (end 91.44 106.68) (width 0.2032) (layer "F.Cu") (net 7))
 (segment (start 96.52 114.3) (end 101.6 114.3) (width 0.2032) (layer "F.Cu") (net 7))
 (segment (start 88.9 109.22) (end 91.44 109.22) (width 0.25) (layer "F.Cu") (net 7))
 (segment (start 93.98 111.76) (end 96.52 114.3) (width 0.2032) (layer "F.Cu") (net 7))
 (segment (start 91.44 116.84) (end 99.06 116.84) (width 0.25) (layer "F.Cu") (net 5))
 (segment (start 88.9 114.1) (end 91.44 116.64) (width 0.25) (layer "F.Cu") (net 5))
 (segment (start 88.9 118.43) (end 88.9 114.1) (width 0.25) (layer "F.Cu") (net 5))
 (segment (start 89.85 119.38) (end 93.03 119.38) (width 0.25) (layer "F.Cu") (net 5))
 (segment (start 91.44 116.64) (end 91.44 116.84) (width 0.25) (layer "F.Cu") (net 5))
 (segment (start 88.9 118.43) (end 89.85 119.38) (width 0.25) (layer "F.Cu") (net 5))
 (segment (start 99.06 116.84) (end 101.1968 116.84) (width 0.2032) (layer "F.Cu") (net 5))
 (segment (start 116.84 117.7525) (end 116.84 117.4464) (width 0.2032) (layer "F.Cu") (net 11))
 (segment (start 116.84 117.4464) (end 119.9864 117.4464) (width 0.2032) (layer "F.Cu") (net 11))
 (segment (start 124.46 116.84) (end 127 116.84) (width 0.2032) (layer "F.Cu") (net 11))
 (segment (start 115.2125 119.38) (end 116.84 117.7525) (width 0.2032) (layer "F.Cu") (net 11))
 (segment (start 121.92 119.38) (end 124.46 116.84) (width 0.2032) (layer "F.Cu") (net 11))
 (segment (start 119.9864 117.4464) (end 121.92 119.38) (width 0.2032) (layer "F.Cu") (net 11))
 (via (at 127 116.84) (size 0.8) (drill 0.4) (layers "F.Cu" "B.Cu") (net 11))
 (segment (start 127 116.84) (end 129.54 119.38) (width 0.2032) (layer "B.Cu") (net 11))
 (segment (start 115.2125 121.92) (end 121.92 121.92) (width 0.2032) (layer "F.Cu") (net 12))
 (via (at 121.92 121.92) (size 0.8) (drill 0.4) (layers "F.Cu" "B.Cu") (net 12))
 (segment (start 122.682 121.158) (end 128.016 121.158) (width 0.2032) (layer "B.Cu") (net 12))
 (segment (start 121.92 121.92) (end 122.682 121.158) (width 0.2032) (layer "B.Cu") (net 12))
 (segment (start 117.7525 127) (end 121.92 127) (width 0.2032) (layer "F.Cu") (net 13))
 (segment (start 115.2125 124.46) (end 117.7525 127) (width 0.2032) (layer "F.Cu") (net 13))
 (segment (start 121.92 127) (end 124.46 124.46) (width 0.2032) (layer "F.Cu") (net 13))
 (via (at 124.46 124.46) (size 0.8) (drill 0.4) (layers "F.Cu" "B.Cu") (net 13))
 (segment (start 126.238 122.682) (end 129.54 122.682) (width 0.2032) (layer "B.Cu") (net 13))
 (segment (start 124.46 124.46) (end 126.238 122.682) (width 0.2032) (layer "B.Cu") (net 13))
 (segment (start 101.6 81.28) (end 109.22 81.28) (width 0.6096) (layer "F.Cu") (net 10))
 (segment (start 99.98 82.9) (end 99.98 85.4025) (width 0.6096) (layer "F.Cu") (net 10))
 (segment (start 101.6 81.28) (end 99.98 82.9) (width 0.6096) (layer "F.Cu") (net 10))
 (segment (start 109.22 81.28) (end 111.76 83.82) (width 0.6096) (layer "F.Cu") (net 10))
 (segment (start 113.94 95.98) (end 119.74 95.98) (width 0.2032) (layer "F.Cu") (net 15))
 (segment (start 114.3 101.8616) (end 113.94 101.5016) (width 0.2032) (layer "F.Cu") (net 15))
 (segment (start 114.3 111.76) (end 114.3 101.8616) (width 0.2032) (layer "F.Cu") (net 15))
 (segment (start 113.94 101.5016) (end 113.94 95.98) (width 0.2032) (layer "F.Cu") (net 15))
 (segment (start 111.18979 119.38) (end 109.22 119.38) (width 0.2032) (layer "B.Cu") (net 15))
 (segment (start 111.474895 114.585105) (end 111.474895 119.094895) (width 0.2032) (layer "B.Cu") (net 15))
 (segment (start 114.3 111.76) (end 111.474895 114.585105) (width 0.2032) (layer "B.Cu") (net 15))
 (segment (start 111.474895 119.094895) (end 111.18979 119.38) (width 0.2032) (layer "B.Cu") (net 15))
 (segment (start 121.56 101.06) (end 124.1 101.06) (width 0.25) (layer "F.Cu") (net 6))
 (segment (start 124.1 101.06) (end 129.9 101.06) (width 0.2032) (layer "F.Cu") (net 6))
 (segment (start 121.56 101.06) (end 121.56 107.04) (width 0.2032) (layer "F.Cu") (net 6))
 (segment (start 121.56 107.04) (end 116.84 111.76) (width 0.2032) (layer "F.Cu") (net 6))
 (segment (start 109.22 116.84) (end 111.071695 114.988305) (width 0.2032) (layer "B.Cu") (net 6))
 (segment (start 111.071695 114.988305) (end 111.071695 112.448305) (width 0.2032) (layer "B.Cu") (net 6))
 (segment (start 112.9116 110.6084) (end 115.6884 110.6084) (width 0.2032) (layer "B.Cu") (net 6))
 (segment (start 115.6884 110.6084) (end 116.84 111.76) (width 0.2032) (layer "B.Cu") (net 6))
 (segment (start 111.071695 112.448305) (end 112.9116 110.6084) (width 0.2032) (layer "B.Cu") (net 6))
 (segment (start 107.7816 115.7384) (end 104.14 112.0968) (width 0.2032) (layer "F.Cu") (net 21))
 (segment (start 113.3875 116.84) (end 113.3875 119.38) (width 0.25) (layer "F.Cu") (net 21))
 (segment (start 104.14 106.68) (end 101.6 104.14) (width 0.25) (layer "F.Cu") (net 21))
 (segment (start 113.3875 116.84) (end 112.2859 115.7384) (width 0.2032) (layer "F.Cu") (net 21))
 (segment (start 104.14 112.0968) (end 104.14 106.68) (width 0.25) (layer "F.Cu") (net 21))
 (segment (start 112.2859 115.7384) (end 107.7816 115.7384) (width 0.2032) (layer "F.Cu") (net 21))
 (segment (start 106.68 119.38) (end 101.6 119.38) (width 0.2032) (layer "F.Cu") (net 17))
 (segment (start 113.3875 121.92) (end 111.114698 121.92) (width 0.2032) (layer "F.Cu") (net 17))
 (segment (start 109.676298 120.4816) (end 107.7816 120.4816) (width 0.2032) (layer "F.Cu") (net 17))
 (segment (start 111.114698 121.92) (end 109.676298 120.4816) (width 0.2032) (layer "F.Cu") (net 17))
 (segment (start 107.7816 120.4816) (end 106.68 119.38) (width 0.2032) (layer "F.Cu") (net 17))
 (segment (start 111.76 124.46) (end 110.6584 123.3584) (width 0.2032) (layer "F.Cu") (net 16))
 (segment (start 110.6584 123.3584) (end 105.5784 123.3584) (width 0.2032) (layer "F.Cu") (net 16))
 (segment (start 105.5784 123.3584) (end 104.14 121.92) (width 0.2032) (layer "F.Cu") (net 16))
 (segment (start 104.14 121.92) (end 101.6 121.92) (width 0.2032) (layer "F.Cu") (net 16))
 (segment (start 111.76 124.46) (end 113.3875 124.46) (width 0.2032) (layer "F.Cu") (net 16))
 (segment (start 117.9916 113.1484) (end 113.3852 113.1484) (width 0.2032) (layer "F.Cu") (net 9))
 (segment (start 106.68 109.22) (end 106.68 96.52) (width 0.2032) (layer "F.Cu") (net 9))
 (segment (start 119.38 111.76) (end 117.9916 113.1484) (width 0.2032) (layer "F.Cu") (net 9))
 (segment (start 99.9725 93.98) (end 99.06 94.8925) (width 0.2032) (layer "F.Cu") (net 9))
 (segment (start 106.68 96.52) (end 104.14 93.98) (width 0.2032) (layer "F.Cu") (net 9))
 (segment (start 104.14 93.98) (end 101.6 93.98) (width 0.2032) (layer "F.Cu") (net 9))
 (segment (start 110.8952 110.6584) (end 108.1184 110.6584) (width 0.2032) (layer "F.Cu") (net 9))
 (segment (start 108.1184 110.6584) (end 106.68 109.22) (width 0.2032) (layer "F.Cu") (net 9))
 (segment (start 101.6 93.98) (end 99.9725 93.98) (width 0.2032) (layer "F.Cu") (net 9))
 (segment (start 113.3852 113.1484) (end 110.8952 110.6584) (width 0.2032) (layer "F.Cu") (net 9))
 (segment (start 124.1 111.22) (end 122.46 111.22) (width 0.2032) (layer "F.Cu") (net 14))
 (segment (start 116.84 114.3) (end 117.317009 113.822991) (width 0.2032) (layer "F.Cu") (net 14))
 (segment (start 120.194304 113.485696) (end 119.857009 113.148401) (width 0.2032) (layer "F.Cu") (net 14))
 (segment (start 118.66619 113.148401) (end 117.9916 113.822991) (width 0.2032) (layer "F.Cu") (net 14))
 (segment (start 117.317009 113.822991) (end 117.9916 113.822991) (width 0.2032) (layer "F.Cu") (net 14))
 (segment (start 124.1 111.22) (end 129.9 111.22) (width 0.2032) (layer "F.Cu") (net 14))
 (segment (start 119.857009 113.148401) (end 118.66619 113.148401) (width 0.2032) (layer "F.Cu") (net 14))
 (segment (start 122.46 111.22) (end 120.194304 113.485696) (width 0.2032) (layer "F.Cu") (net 14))
 (segment (start 116.84 114.3) (end 109.22 121.92) (width 0.2032) (layer "B.Cu") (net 14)))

